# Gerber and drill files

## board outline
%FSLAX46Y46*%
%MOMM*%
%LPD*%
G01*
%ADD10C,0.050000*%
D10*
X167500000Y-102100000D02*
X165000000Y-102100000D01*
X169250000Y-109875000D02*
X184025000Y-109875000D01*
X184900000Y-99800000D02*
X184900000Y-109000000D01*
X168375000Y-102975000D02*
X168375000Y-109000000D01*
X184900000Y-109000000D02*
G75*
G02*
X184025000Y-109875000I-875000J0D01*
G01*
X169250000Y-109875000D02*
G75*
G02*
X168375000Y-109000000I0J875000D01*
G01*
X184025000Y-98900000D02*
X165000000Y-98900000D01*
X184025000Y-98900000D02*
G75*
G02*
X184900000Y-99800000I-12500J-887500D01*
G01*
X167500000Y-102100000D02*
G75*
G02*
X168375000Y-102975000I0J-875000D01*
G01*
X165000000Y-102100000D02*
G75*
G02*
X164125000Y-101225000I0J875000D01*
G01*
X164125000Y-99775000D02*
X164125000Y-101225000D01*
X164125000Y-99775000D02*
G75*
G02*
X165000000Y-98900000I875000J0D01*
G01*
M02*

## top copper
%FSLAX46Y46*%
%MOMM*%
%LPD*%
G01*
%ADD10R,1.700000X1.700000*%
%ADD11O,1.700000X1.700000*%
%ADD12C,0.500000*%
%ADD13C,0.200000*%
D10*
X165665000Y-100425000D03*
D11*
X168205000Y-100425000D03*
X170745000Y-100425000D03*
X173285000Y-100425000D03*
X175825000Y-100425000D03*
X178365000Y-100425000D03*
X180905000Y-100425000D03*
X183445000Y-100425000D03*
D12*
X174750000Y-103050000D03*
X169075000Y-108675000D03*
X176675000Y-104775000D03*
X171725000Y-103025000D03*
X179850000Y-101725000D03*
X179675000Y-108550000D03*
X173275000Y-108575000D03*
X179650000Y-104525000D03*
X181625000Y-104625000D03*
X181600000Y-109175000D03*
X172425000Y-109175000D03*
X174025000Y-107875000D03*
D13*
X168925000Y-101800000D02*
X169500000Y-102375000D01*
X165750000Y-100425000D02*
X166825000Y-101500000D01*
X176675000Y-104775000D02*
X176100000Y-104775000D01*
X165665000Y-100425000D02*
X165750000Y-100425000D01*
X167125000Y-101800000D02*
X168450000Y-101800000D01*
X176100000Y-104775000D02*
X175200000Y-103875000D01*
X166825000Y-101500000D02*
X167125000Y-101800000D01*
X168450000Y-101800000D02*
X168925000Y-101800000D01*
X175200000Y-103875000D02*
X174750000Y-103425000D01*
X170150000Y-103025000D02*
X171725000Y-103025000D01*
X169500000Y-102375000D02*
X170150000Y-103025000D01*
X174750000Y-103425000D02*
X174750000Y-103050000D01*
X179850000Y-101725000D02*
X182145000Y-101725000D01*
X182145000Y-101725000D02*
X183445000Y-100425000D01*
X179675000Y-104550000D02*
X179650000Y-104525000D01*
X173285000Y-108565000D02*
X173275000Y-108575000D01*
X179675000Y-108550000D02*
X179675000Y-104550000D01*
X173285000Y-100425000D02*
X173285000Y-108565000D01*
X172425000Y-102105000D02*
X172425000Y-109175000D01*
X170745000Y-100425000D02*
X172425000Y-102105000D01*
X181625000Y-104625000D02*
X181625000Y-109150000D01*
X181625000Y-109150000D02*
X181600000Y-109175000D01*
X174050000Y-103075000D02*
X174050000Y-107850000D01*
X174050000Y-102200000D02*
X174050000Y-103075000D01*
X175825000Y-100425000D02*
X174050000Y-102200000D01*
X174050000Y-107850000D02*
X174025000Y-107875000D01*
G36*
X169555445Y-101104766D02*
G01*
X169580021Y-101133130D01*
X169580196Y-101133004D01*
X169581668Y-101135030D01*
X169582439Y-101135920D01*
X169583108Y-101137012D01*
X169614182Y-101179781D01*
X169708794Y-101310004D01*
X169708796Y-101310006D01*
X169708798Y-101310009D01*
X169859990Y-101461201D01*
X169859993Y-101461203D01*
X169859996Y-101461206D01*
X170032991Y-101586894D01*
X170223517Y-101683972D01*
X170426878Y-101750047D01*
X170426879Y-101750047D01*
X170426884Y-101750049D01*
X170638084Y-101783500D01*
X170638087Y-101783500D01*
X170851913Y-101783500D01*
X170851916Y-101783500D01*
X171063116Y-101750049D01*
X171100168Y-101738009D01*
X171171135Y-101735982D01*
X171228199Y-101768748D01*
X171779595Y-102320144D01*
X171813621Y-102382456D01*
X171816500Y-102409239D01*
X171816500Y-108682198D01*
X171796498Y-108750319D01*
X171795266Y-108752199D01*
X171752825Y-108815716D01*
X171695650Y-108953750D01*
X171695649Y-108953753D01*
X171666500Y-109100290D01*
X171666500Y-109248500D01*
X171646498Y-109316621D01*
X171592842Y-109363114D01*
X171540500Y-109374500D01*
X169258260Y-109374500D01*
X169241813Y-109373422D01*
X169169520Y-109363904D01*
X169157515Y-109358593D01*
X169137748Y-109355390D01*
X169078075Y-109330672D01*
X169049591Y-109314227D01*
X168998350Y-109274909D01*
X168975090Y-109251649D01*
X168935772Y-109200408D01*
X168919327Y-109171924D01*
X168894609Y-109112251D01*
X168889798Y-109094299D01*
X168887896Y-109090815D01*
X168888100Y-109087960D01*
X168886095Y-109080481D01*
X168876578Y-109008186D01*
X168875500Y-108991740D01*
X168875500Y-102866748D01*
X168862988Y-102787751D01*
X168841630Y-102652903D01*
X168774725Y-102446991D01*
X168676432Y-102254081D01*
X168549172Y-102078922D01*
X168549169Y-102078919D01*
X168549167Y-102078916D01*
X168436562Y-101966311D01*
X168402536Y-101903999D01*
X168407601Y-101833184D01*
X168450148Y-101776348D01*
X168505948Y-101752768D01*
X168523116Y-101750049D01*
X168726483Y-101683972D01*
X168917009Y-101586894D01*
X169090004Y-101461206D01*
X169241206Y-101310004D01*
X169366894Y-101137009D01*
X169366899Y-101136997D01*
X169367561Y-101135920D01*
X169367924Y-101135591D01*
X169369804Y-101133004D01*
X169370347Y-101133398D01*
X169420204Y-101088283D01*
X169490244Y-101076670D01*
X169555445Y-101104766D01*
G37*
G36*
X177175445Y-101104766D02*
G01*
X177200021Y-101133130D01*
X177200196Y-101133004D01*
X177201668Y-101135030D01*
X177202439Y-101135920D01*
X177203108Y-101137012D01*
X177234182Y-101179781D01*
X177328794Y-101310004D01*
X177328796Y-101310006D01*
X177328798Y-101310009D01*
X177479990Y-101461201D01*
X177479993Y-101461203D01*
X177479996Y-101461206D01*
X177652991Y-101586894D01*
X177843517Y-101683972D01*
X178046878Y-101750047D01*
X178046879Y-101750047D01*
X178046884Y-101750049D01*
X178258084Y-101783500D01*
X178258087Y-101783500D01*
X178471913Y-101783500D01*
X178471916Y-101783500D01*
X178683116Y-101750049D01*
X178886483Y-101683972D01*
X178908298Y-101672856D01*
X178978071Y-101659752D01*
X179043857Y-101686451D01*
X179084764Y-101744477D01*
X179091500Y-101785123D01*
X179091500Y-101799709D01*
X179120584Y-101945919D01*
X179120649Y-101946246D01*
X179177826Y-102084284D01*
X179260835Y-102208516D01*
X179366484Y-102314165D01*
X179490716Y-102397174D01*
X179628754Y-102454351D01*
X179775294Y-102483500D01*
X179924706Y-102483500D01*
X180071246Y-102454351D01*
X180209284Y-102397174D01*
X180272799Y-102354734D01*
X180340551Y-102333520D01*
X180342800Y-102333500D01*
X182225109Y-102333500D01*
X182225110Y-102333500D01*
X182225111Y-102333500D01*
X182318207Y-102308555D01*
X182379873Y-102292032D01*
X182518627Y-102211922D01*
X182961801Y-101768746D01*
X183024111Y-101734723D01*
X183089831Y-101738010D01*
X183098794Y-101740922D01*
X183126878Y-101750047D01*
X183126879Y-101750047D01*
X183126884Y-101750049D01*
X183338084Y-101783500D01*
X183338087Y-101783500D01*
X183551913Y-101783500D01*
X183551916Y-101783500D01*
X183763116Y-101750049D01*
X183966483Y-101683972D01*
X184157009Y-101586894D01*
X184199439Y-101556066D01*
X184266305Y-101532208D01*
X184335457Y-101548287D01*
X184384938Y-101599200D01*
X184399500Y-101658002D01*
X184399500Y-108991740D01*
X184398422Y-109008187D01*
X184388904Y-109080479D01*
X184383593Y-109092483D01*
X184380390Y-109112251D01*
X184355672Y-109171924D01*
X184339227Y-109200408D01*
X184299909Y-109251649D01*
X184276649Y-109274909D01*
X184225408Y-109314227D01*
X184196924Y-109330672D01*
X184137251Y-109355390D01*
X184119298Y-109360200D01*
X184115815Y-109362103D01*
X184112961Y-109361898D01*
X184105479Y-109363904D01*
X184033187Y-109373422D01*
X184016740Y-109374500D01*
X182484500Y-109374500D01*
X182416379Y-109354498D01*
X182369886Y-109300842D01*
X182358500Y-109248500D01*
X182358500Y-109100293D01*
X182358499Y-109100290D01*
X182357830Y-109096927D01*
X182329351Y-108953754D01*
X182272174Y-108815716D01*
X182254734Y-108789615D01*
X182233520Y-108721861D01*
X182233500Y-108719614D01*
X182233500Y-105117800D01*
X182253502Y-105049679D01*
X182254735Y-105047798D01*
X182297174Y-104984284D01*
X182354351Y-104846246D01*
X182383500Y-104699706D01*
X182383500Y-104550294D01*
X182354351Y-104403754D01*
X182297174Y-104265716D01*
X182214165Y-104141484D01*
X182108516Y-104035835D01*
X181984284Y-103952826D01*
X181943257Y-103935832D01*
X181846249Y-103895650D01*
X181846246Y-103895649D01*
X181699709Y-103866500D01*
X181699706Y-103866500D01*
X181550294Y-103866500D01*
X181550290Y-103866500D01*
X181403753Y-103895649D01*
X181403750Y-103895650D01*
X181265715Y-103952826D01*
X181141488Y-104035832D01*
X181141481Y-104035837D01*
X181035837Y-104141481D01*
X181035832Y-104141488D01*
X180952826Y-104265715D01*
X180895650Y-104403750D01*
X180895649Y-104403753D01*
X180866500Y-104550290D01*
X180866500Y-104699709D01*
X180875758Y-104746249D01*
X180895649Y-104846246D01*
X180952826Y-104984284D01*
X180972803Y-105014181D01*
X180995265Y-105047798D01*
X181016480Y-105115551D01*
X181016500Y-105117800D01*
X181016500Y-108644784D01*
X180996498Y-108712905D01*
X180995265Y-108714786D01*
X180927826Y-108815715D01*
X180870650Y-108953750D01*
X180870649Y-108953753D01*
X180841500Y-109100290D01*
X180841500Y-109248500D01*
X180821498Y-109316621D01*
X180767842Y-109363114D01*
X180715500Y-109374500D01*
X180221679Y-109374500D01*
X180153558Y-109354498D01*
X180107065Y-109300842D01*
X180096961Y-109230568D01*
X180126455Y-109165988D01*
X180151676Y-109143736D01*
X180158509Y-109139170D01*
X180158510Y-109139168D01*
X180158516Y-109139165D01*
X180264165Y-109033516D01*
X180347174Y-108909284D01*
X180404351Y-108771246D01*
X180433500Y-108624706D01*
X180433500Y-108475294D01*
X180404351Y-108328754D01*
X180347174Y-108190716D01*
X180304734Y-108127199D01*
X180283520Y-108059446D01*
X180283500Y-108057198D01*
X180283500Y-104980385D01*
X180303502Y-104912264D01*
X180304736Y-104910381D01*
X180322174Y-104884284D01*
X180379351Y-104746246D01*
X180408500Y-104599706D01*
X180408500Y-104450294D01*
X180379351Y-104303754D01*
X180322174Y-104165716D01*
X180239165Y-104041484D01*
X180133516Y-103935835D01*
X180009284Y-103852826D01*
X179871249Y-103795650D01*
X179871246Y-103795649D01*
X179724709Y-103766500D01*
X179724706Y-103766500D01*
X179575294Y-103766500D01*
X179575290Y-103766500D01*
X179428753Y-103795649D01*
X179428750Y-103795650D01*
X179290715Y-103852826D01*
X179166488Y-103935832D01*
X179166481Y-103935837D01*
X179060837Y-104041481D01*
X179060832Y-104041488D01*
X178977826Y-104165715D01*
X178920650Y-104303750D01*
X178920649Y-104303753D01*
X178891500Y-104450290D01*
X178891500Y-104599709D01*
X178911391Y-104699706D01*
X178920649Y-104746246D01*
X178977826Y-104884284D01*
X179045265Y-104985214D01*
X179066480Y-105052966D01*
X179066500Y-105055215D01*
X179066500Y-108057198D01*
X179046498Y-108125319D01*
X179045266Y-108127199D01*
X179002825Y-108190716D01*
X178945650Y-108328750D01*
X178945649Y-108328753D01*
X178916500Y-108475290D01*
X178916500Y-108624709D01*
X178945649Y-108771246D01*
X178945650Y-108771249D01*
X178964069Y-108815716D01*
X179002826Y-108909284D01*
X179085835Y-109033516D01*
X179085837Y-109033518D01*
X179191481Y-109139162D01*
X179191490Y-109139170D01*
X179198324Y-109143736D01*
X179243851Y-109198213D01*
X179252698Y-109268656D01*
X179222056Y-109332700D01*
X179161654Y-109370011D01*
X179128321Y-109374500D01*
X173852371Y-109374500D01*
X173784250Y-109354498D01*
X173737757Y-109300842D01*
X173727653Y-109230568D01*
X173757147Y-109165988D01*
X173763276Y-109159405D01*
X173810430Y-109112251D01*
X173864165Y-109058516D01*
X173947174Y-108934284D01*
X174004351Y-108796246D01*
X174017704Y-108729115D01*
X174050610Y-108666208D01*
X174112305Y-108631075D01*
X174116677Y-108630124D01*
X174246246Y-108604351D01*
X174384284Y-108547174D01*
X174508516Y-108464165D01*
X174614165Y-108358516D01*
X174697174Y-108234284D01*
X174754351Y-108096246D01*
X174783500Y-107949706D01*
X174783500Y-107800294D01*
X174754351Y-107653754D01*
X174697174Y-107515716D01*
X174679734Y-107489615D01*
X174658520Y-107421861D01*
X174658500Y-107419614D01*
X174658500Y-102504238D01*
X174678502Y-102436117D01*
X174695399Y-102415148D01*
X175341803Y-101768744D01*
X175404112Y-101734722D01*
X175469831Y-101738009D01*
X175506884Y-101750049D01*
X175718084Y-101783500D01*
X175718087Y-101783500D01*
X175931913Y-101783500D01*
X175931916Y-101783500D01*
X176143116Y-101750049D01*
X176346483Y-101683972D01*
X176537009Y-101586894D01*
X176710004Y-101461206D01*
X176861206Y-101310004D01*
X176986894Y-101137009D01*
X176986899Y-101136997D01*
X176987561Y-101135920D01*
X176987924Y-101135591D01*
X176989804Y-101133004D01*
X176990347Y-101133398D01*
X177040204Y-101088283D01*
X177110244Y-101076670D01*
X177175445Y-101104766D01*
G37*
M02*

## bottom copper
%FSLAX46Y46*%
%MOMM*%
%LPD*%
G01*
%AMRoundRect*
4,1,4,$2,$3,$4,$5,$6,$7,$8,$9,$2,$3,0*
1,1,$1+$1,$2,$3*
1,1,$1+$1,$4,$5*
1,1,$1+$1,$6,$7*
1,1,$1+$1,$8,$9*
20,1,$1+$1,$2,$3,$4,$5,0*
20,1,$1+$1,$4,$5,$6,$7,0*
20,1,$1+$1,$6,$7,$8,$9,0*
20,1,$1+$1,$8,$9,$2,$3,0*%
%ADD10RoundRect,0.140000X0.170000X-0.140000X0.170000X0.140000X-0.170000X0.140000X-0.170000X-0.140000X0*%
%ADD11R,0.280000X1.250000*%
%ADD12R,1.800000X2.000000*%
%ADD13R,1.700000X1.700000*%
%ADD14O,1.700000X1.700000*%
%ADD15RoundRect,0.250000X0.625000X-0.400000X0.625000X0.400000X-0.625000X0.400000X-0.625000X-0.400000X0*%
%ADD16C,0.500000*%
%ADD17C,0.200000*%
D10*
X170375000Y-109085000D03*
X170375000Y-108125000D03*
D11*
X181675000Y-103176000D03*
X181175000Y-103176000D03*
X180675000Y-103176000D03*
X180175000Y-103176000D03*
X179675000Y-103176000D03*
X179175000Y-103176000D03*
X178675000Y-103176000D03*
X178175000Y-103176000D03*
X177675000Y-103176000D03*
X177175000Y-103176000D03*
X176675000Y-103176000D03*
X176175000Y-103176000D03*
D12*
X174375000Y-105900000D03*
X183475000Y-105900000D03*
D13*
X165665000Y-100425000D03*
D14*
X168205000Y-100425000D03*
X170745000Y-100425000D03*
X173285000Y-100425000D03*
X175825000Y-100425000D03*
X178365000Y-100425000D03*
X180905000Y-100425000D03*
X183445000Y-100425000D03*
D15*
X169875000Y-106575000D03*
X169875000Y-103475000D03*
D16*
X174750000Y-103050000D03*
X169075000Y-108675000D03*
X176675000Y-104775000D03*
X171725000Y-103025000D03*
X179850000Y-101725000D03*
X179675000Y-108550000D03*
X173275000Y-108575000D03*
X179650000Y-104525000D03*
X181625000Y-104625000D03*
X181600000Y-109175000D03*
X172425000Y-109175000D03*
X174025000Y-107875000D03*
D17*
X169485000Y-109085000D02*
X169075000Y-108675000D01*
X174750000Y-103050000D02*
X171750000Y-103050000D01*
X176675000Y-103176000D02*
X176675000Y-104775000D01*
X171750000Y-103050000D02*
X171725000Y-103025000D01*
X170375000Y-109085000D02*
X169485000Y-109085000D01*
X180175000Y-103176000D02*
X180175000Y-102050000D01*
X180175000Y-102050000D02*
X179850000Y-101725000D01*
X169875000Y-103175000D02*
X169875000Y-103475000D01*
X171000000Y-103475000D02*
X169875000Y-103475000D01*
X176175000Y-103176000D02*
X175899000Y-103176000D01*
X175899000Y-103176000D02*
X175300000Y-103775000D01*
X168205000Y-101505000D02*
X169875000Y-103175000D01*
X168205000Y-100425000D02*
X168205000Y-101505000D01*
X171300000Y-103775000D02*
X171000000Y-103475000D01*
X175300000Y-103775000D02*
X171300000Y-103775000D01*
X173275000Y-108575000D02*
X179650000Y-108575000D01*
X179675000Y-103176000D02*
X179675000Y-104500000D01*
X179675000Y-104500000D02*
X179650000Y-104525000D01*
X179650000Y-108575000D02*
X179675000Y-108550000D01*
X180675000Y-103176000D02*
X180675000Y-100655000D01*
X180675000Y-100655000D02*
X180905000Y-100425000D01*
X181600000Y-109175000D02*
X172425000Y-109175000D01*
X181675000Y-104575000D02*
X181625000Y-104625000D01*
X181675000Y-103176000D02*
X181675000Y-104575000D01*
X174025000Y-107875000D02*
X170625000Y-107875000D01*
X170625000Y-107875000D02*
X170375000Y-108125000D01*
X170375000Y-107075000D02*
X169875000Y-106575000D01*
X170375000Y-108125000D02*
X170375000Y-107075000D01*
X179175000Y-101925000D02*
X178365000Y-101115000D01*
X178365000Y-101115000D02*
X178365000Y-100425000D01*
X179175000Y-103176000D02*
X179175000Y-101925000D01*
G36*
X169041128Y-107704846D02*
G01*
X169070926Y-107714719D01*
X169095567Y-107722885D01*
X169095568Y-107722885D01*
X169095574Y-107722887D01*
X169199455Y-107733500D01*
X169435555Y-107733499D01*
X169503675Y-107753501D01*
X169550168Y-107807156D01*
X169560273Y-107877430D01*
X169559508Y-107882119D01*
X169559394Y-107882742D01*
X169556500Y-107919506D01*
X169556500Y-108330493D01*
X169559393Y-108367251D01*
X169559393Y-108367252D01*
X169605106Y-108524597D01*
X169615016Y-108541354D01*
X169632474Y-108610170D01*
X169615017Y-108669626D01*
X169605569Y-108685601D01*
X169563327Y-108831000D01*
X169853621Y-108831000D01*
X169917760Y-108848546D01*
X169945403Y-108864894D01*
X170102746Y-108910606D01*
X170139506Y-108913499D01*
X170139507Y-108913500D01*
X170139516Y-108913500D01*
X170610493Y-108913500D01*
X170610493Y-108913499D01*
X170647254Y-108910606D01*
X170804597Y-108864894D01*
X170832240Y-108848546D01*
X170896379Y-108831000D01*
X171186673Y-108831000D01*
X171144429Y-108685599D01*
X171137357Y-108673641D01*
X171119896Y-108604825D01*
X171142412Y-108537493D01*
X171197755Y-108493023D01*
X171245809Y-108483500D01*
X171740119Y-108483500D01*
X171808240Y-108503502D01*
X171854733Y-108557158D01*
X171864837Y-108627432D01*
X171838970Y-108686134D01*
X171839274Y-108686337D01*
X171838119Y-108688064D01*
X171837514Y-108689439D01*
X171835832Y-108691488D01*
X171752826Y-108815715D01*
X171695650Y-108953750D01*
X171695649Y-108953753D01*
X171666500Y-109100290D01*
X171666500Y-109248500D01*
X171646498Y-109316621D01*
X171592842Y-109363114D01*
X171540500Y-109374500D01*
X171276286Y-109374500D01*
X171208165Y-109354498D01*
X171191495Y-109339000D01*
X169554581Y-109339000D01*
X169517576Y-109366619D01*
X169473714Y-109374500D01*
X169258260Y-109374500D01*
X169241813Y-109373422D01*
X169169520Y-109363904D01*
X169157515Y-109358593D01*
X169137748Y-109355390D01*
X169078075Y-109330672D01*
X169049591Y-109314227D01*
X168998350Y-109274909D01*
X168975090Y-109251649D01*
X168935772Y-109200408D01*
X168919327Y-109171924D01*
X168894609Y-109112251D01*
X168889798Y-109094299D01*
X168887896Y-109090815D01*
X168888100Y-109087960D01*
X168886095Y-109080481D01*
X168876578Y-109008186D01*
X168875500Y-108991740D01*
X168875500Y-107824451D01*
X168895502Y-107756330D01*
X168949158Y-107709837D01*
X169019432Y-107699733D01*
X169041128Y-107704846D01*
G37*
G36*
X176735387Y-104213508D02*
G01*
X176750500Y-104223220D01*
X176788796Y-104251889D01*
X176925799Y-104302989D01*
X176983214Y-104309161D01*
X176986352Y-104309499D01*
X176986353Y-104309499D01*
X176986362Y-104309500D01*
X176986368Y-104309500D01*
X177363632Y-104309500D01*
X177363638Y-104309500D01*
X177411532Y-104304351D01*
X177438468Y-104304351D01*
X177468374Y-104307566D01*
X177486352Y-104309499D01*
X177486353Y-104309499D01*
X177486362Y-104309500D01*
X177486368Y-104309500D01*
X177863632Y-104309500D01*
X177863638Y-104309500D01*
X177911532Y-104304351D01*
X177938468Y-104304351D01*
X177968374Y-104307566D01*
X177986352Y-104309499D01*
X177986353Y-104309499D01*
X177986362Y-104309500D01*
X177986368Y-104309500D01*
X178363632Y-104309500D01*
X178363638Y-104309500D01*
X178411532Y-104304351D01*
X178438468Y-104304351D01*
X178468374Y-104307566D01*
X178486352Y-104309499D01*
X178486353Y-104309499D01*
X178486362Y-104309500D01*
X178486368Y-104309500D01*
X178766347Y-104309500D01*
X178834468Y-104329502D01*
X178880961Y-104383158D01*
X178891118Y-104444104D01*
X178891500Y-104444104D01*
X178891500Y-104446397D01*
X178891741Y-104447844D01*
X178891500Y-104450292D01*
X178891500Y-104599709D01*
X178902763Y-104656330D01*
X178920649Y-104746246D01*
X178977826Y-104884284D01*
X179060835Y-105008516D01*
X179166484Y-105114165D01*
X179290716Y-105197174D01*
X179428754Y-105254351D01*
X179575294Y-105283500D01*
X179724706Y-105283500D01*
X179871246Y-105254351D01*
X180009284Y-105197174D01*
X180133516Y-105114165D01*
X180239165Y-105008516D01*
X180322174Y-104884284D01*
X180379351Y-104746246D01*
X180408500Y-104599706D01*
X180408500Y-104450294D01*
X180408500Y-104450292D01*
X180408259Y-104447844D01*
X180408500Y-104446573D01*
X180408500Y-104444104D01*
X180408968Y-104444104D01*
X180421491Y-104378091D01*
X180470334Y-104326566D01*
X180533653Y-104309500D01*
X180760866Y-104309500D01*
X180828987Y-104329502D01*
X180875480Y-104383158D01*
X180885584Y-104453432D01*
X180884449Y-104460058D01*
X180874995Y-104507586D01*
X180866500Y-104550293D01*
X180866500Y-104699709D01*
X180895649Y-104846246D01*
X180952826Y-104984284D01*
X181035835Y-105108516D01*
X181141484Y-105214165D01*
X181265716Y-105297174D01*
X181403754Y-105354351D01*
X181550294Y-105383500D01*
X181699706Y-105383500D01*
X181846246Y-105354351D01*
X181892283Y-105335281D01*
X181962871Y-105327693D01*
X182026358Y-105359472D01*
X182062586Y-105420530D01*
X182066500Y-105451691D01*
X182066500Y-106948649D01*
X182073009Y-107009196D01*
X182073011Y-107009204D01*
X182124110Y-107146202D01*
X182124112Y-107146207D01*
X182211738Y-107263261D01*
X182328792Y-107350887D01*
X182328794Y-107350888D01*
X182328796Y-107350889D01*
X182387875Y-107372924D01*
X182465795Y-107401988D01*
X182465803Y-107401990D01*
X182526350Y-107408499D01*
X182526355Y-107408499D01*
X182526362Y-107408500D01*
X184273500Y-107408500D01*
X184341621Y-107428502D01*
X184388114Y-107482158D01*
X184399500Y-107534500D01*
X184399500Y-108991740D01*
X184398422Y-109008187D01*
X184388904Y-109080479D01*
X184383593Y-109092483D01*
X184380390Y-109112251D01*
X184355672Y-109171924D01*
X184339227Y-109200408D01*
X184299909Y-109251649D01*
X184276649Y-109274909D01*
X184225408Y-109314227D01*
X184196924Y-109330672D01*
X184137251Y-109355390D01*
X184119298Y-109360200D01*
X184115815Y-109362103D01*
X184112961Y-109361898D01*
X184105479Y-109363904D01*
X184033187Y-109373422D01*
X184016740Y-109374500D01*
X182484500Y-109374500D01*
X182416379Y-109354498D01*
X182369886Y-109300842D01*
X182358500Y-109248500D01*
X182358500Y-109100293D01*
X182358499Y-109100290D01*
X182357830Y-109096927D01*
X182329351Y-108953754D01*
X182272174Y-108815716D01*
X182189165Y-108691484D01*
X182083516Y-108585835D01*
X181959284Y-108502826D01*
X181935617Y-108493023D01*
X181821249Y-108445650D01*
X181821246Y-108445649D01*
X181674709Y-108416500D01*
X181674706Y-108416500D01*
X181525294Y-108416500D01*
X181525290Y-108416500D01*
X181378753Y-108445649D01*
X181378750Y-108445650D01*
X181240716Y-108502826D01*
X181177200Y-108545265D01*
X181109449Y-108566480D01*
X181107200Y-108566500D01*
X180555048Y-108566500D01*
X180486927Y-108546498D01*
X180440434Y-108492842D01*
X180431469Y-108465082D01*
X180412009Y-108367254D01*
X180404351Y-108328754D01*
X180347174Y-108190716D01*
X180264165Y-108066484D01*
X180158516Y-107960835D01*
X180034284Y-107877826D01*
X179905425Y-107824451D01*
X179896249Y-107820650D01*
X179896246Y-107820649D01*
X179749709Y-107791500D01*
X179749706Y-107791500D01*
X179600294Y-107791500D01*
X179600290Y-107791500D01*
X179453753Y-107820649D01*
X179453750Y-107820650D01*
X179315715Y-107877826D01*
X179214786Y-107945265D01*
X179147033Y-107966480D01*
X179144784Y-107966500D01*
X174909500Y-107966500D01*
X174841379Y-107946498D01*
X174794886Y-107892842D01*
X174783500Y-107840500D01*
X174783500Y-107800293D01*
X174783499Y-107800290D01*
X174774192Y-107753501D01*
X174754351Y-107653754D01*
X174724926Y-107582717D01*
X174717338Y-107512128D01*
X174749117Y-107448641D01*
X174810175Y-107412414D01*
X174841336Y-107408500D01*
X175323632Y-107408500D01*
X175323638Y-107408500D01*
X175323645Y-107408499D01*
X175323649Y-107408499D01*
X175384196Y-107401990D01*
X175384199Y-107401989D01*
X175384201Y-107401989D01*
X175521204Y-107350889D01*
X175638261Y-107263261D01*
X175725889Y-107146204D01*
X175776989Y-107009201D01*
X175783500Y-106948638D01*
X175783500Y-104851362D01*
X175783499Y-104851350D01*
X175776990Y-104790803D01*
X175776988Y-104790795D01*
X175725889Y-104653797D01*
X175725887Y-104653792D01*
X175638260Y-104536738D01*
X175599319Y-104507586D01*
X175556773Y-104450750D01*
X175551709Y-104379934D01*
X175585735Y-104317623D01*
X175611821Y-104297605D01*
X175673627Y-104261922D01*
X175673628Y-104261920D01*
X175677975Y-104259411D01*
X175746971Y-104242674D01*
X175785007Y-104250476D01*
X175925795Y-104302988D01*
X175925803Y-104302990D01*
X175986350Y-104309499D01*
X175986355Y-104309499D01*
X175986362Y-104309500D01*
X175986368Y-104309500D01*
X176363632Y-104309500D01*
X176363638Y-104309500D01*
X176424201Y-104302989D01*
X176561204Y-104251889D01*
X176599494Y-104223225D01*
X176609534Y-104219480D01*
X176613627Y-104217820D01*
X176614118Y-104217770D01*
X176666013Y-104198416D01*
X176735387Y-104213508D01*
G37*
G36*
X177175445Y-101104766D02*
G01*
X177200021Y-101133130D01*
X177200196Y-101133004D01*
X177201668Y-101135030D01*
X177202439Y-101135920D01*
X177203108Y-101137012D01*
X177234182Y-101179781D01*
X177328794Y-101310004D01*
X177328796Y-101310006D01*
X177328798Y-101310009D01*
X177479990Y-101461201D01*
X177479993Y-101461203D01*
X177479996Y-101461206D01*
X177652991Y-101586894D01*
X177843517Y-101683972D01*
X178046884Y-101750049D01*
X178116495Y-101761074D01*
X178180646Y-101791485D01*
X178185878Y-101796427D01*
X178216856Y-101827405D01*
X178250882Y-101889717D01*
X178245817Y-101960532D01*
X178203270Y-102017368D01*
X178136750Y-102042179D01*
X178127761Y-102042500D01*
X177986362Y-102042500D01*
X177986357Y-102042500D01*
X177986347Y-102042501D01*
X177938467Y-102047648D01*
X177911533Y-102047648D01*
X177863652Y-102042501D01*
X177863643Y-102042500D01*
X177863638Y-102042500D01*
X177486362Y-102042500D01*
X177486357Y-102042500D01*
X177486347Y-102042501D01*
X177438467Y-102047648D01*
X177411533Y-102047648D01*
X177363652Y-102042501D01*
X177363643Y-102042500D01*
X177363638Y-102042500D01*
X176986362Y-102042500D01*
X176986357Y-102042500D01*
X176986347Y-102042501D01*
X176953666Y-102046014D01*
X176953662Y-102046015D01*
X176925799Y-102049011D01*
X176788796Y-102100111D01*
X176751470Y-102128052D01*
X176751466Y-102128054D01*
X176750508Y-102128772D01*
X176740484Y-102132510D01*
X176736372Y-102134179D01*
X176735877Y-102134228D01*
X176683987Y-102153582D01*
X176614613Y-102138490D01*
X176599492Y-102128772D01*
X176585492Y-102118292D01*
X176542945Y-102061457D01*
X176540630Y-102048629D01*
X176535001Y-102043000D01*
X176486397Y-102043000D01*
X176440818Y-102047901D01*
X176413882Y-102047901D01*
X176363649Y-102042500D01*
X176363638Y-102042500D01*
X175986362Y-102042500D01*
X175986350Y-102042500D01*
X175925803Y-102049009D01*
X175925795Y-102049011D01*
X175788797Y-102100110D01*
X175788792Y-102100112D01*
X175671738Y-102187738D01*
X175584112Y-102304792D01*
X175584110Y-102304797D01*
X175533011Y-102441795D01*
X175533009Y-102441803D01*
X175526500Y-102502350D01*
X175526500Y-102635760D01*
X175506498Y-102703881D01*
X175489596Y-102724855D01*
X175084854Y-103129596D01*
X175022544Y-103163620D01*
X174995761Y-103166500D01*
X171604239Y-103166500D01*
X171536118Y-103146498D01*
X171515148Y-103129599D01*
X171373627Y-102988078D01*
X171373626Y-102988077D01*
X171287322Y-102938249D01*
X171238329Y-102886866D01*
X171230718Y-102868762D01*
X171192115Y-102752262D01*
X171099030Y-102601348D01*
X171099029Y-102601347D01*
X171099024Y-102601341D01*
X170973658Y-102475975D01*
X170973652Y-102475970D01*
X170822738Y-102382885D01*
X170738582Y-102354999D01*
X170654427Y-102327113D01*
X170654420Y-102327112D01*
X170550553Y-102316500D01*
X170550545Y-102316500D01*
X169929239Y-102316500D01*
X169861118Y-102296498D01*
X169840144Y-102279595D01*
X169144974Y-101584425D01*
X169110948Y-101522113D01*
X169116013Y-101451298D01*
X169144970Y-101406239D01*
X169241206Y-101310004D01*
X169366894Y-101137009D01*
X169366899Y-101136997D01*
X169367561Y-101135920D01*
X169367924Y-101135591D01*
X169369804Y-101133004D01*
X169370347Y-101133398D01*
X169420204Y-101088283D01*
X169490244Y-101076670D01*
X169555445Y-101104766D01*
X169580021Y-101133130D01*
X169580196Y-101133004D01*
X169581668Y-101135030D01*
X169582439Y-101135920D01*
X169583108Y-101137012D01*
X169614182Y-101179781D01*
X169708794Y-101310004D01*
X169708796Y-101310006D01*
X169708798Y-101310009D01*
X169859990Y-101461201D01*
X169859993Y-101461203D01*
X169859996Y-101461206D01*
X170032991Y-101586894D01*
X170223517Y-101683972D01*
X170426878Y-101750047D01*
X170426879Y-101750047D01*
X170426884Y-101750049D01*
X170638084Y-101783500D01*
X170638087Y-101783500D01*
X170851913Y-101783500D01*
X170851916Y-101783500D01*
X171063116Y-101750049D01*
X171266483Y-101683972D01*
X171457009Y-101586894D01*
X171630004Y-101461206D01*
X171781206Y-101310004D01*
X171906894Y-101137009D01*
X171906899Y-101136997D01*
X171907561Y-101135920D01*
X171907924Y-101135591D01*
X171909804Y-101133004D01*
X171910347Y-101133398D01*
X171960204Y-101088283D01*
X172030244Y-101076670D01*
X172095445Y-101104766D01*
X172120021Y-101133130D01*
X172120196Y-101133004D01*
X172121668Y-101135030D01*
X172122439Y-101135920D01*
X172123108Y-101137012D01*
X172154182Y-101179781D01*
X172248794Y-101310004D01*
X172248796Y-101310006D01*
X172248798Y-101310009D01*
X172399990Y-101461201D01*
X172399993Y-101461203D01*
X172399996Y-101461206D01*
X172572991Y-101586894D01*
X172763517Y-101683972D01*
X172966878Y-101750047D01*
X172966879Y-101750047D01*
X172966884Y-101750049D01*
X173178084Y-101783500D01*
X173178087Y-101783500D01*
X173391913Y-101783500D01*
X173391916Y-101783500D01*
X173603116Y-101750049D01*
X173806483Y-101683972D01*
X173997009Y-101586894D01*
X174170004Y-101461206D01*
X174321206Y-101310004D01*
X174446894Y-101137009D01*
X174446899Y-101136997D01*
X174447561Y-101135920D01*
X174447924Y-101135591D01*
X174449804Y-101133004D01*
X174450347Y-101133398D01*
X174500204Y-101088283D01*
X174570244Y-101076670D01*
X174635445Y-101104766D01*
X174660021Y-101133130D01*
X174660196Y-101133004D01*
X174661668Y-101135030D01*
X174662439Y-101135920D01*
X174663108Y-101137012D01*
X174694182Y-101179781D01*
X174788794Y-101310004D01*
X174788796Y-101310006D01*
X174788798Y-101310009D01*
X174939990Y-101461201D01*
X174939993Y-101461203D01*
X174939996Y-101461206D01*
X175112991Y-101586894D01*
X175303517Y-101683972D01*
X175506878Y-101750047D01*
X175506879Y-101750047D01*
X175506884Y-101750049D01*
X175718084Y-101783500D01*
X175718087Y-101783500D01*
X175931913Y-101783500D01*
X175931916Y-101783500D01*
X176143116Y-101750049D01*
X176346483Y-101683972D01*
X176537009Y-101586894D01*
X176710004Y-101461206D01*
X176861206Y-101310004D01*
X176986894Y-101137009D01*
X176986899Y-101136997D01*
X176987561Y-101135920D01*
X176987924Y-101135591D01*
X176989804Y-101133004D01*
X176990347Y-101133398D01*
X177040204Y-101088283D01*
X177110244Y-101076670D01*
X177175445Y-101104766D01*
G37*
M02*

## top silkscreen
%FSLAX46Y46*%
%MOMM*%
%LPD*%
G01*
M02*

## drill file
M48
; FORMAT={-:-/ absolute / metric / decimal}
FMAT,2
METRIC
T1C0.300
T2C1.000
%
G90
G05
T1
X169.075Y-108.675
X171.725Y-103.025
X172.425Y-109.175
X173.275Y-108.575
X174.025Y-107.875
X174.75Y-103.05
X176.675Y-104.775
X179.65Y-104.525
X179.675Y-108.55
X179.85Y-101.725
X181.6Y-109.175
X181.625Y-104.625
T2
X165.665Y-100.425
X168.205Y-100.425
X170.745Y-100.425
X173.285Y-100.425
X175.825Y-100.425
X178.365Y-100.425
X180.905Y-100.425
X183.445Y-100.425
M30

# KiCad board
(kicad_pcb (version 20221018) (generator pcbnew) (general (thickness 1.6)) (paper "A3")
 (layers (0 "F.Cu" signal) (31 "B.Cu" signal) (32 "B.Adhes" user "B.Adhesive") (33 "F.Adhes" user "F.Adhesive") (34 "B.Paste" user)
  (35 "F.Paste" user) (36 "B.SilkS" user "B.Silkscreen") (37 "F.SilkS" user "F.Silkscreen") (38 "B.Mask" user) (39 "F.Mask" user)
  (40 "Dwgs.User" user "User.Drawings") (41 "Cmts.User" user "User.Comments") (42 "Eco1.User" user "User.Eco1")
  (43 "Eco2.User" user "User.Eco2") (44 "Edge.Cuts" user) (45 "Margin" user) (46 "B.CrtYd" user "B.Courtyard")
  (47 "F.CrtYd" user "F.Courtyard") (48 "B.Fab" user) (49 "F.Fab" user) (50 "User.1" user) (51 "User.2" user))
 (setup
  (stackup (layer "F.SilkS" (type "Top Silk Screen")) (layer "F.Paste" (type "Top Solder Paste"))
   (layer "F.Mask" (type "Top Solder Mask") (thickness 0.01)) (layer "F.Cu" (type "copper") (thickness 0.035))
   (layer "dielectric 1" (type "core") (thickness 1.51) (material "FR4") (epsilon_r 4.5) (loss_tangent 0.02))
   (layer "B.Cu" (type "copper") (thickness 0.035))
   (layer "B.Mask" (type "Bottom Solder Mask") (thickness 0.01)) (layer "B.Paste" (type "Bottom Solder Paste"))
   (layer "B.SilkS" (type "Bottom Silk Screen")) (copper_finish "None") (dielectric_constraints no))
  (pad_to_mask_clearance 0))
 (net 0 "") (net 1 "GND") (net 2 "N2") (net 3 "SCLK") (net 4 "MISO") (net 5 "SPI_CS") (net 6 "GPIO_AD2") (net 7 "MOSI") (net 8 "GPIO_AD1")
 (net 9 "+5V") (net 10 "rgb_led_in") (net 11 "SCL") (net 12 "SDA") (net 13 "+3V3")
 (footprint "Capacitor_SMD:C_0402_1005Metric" (layer "B.Cu") (at 170.375 108.605 90)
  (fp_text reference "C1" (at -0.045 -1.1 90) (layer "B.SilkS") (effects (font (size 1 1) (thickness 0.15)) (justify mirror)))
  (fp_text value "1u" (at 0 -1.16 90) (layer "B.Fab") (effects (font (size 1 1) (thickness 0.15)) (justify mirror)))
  (pad "1" smd roundrect (at -0.48 0 90) (size 0.56 0.62) (layers "B.Cu" "B.Paste" "B.Mask") (roundrect_rratio 0.25) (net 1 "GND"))
  (pad "2" smd roundrect (at 0.48 0 90) (size 0.56 0.62) (layers "B.Cu" "B.Paste" "B.Mask") (roundrect_rratio 0.25) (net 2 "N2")))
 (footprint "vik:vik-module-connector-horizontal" (layer "B.Cu") (at 178.925 105.214 180)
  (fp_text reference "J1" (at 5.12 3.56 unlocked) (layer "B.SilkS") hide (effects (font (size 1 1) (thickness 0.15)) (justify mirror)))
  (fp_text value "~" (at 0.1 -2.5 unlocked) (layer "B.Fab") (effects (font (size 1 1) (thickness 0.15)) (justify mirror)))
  (pad "1" smd rect (at -2.75 2.038 180) (size 0.28 1.25) (layers "B.Cu" "B.Paste" "B.Mask") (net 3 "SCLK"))
  (pad "2" smd rect (at -2.25 2.038 180) (size 0.28 1.25) (layers "B.Cu" "B.Paste" "B.Mask") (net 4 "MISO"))
  (pad "3" smd rect (at -1.75 2.038 180) (size 0.28 1.25) (layers "B.Cu" "B.Paste" "B.Mask") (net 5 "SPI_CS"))
  (pad "4" smd rect (at -1.25 2.038 180) (size 0.28 1.25) (layers "B.Cu" "B.Paste" "B.Mask") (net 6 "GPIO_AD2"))
  (pad "5" smd rect (at -0.75 2.038 180) (size 0.28 1.25) (layers "B.Cu" "B.Paste" "B.Mask") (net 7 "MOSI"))
  (pad "6" smd rect (at -0.25 2.038 180) (size 0.28 1.25) (layers "B.Cu" "B.Paste" "B.Mask") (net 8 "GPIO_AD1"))
  (pad "7" smd rect (at 0.25 2.038 180) (size 0.28 1.25) (layers "B.Cu" "B.Paste" "B.Mask") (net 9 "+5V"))
  (pad "8" smd rect (at 0.75 2.038 180) (size 0.28 1.25) (layers "B.Cu" "B.Paste" "B.Mask") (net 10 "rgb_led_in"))
  (pad "9" smd rect (at 1.25 2.038 180) (size 0.28 1.25) (layers "B.Cu" "B.Paste" "B.Mask") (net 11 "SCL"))
  (pad "10" smd rect (at 1.75 2.038 180) (size 0.28 1.25) (layers "B.Cu" "B.Paste" "B.Mask") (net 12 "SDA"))
  (pad "11" smd rect (at 2.25 2.038 180) (size 0.28 1.25) (layers "B.Cu" "B.Paste" "B.Mask") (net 1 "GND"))
  (pad "12" smd rect (at 2.75 2.038 180) (size 0.28 1.25) (layers "B.Cu" "B.Paste" "B.Mask") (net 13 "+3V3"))
  (pad "13" smd rect (at 4.55 -0.686 180) (size 1.8 2) (layers "B.Cu" "B.Paste" "B.Mask"))
  (pad "14" smd rect (at -4.55 -0.686 180) (size 1.8 2) (layers "B.Cu" "B.Paste" "B.Mask")))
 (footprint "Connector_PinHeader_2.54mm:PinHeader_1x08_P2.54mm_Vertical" (layer "B.Cu") (at 165.665 100.425 -90)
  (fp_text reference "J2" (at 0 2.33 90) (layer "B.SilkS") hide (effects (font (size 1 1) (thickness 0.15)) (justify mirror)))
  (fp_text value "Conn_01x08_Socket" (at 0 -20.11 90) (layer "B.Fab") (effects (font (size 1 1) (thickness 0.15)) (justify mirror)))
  (pad "1" thru_hole rect (at 0 0 270) (size 1.7 1.7) (drill 1) (layers "*.Cu" "*.Mask") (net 1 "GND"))
  (pad "2" thru_hole oval (at 0 -2.54 270) (size 1.7 1.7) (drill 1) (layers "*.Cu" "*.Mask") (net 13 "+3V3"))
  (pad "3" thru_hole oval (at 0 -5.08 270) (size 1.7 1.7) (drill 1) (layers "*.Cu" "*.Mask") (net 3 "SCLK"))
  (pad "4" thru_hole oval (at 0 -7.62 270) (size 1.7 1.7) (drill 1) (layers "*.Cu" "*.Mask") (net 7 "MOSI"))
  (pad "5" thru_hole oval (at 0 -10.16 270) (size 1.7 1.7) (drill 1) (layers "*.Cu" "*.Mask") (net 2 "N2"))
  (pad "6" thru_hole oval (at 0 -12.7 270) (size 1.7 1.7) (drill 1) (layers "*.Cu" "*.Mask") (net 8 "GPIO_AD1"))
  (pad "7" thru_hole oval (at 0 -15.24 270) (size 1.7 1.7) (drill 1) (layers "*.Cu" "*.Mask") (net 5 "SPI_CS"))
  (pad "8" thru_hole oval (at 0 -17.78 270) (size 1.7 1.7) (drill 1) (layers "*.Cu" "*.Mask") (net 6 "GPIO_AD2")))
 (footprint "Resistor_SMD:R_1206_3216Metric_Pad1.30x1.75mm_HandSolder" (layer "B.Cu") (at 169.875 105.025 90)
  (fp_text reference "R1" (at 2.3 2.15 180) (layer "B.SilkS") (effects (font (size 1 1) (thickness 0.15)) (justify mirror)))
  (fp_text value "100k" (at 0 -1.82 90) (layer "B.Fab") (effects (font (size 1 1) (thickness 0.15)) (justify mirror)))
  (pad "1" smd roundrect (at -1.55 0 90) (size 1.3 1.75) (layers "B.Cu" "B.Paste" "B.Mask") (roundrect_rratio 0.1923076923) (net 2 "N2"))
  (pad "2" smd roundrect (at 1.55 0 90) (size 1.3 1.75) (layers "B.Cu" "B.Paste" "B.Mask") (roundrect_rratio 0.1923076923) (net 13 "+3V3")))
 (gr_line (start 167.5 102.1) (end 165 102.1) (stroke (width 0.05) (type solid)) (layer "Edge.Cuts"))
 (gr_line (start 169.25 109.875) (end 184.025 109.875) (stroke (width 0.05) (type solid)) (layer "Edge.Cuts"))
 (gr_line (start 184.9 99.8) (end 184.9 109) (stroke (width 0.05) (type solid)) (layer "Edge.Cuts"))
 (gr_line (start 168.375 102.975) (end 168.375 109) (stroke (width 0.05) (type solid)) (layer "Edge.Cuts"))
 (gr_arc (start 184.9 109) (mid 184.643718 109.618718) (end 184.025 109.875) (stroke (width 0.05) (type solid)) (layer "Edge.Cuts"))
 (gr_arc (start 169.25 109.875) (mid 168.631282 109.618718) (end 168.375 109) (stroke (width 0.05) (type solid)) (layer "Edge.Cuts"))
 (gr_line (start 184.025 98.9) (end 165 98.9) (stroke (width 0.05) (type solid)) (layer "Edge.Cuts"))
 (gr_arc (start 184.025 98.9) (mid 184.648896 99.168782) (end 184.9 99.8) (stroke (width 0.05) (type solid)) (layer "Edge.Cuts"))
 (gr_arc (start 167.5 102.1) (mid 168.118718 102.356282) (end 168.375 102.975) (stroke (width 0.05) (type solid)) (layer "Edge.Cuts"))
 (gr_arc (start 165 102.1) (mid 164.381282 101.843718) (end 164.125 101.225) (stroke (width 0.05) (type solid)) (layer "Edge.Cuts"))
 (gr_line (start 164.125 99.775) (end 164.125 101.225) (stroke (width 0.05) (type solid)) (layer "Edge.Cuts"))
 (gr_arc (start 164.125 99.775) (mid 164.381282 99.156282) (end 165 98.9) (stroke (width 0.05) (type solid)) (layer "Edge.Cuts"))
 (segment (start 168.925 101.8) (end 169.5 102.375) (width 0.2) (layer "F.Cu") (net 1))
 (segment (start 165.75 100.425) (end 166.825 101.5) (width 0.2) (layer "F.Cu") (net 1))
 (segment (start 176.675 104.775) (end 176.1 104.775) (width 0.2) (layer "F.Cu") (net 1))
 (segment (start 165.665 100.425) (end 165.75 100.425) (width 0.2) (layer "F.Cu") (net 1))
 (segment (start 167.125 101.8) (end 168.45 101.8) (width 0.2) (layer "F.Cu") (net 1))
 (segment (start 176.1 104.775) (end 175.2 103.875) (width 0.2) (layer "F.Cu") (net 1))
 (segment (start 166.825 101.5) (end 167.125 101.8) (width 0.2) (layer "F.Cu") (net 1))
 (segment (start 168.45 101.8) (end 168.925 101.8) (width 0.2) (layer "F.Cu") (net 1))
 (segment (start 175.2 103.875) (end 174.75 103.425) (width 0.2) (layer "F.Cu") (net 1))
 (segment (start 170.15 103.025) (end 171.725 103.025) (width 0.2) (layer "F.Cu") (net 1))
 (segment (start 169.5 102.375) (end 170.15 103.025) (width 0.2) (layer "F.Cu") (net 1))
 (segment (start 174.75 103.425) (end 174.75 103.05) (width 0.2) (layer "F.Cu") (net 1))
 (via (at 174.75 103.05) (size 0.5) (drill 0.3) (layers "F.Cu" "B.Cu") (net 1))
 (via (at 169.075 108.675) (size 0.5) (drill 0.3) (layers "F.Cu" "B.Cu") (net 1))
 (via (at 176.675 104.775) (size 0.5) (drill 0.3) (layers "F.Cu" "B.Cu") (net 1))
 (via (at 171.725 103.025) (size 0.5) (drill 0.3) (layers "F.Cu" "B.Cu") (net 1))
 (segment (start 169.485 109.085) (end 169.075 108.675) (width 0.2) (layer "B.Cu") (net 1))
 (segment (start 174.75 103.05) (end 171.75 103.05) (width 0.2) (layer "B.Cu") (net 1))
 (segment (start 176.675 103.176) (end 176.675 104.775) (width 0.2) (layer "B.Cu") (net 1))
 (segment (start 171.75 103.05) (end 171.725 103.025) (width 0.2) (layer "B.Cu") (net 1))
 (segment (start 170.375 109.085) (end 169.485 109.085) (width 0.2) (layer "B.Cu") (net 1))
 (segment (start 179.85 101.725) (end 182.145 101.725) (width 0.2) (layer "F.Cu") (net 6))
 (segment (start 182.145 101.725) (end 183.445 100.425) (width 0.2) (layer "F.Cu") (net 6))
 (via (at 179.85 101.725) (size 0.5) (drill 0.3) (layers "F.Cu" "B.Cu") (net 6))
 (segment (start 180.175 103.176) (end 180.175 102.05) (width 0.2) (layer "B.Cu") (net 6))
 (segment (start 180.175 102.05) (end 179.85 101.725) (width 0.2) (layer "B.Cu") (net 6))
 (segment (start 169.875 103.175) (end 169.875 103.475) (width 0.2) (layer "B.Cu") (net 13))
 (segment (start 171 103.475) (end 169.875 103.475) (width 0.2) (layer "B.Cu") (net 13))
 (segment (start 176.175 103.176) (end 175.899 103.176) (width 0.2) (layer "B.Cu") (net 13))
 (segment (start 175.899 103.176) (end 175.3 103.775) (width 0.2) (layer "B.Cu") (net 13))
 (segment (start 168.205 101.505) (end 169.875 103.175) (width 0.2) (layer "B.Cu") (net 13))
 (segment (start 168.205 100.425) (end 168.205 101.505) (width 0.2) (layer "B.Cu") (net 13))
 (segment (start 171.3 103.775) (end 171 103.475) (width 0.2) (layer "B.Cu") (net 13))
 (segment (start 175.3 103.775) (end 171.3 103.775) (width 0.2) (layer "B.Cu") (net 13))
 (segment (start 179.675 104.55) (end 179.65 104.525) (width 0.2) (layer "F.Cu") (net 7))
 (segment (start 173.285 108.565) (end 173.275 108.575) (width 0.2) (layer "F.Cu") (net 7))
 (segment (start 179.675 108.55) (end 179.675 104.55) (width 0.2) (layer "F.Cu") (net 7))
 (segment (start 173.285 100.425) (end 173.285 108.565) (width 0.2) (layer "F.Cu") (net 7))
 (via (at 179.675 108.55) (size 0.5) (drill 0.3) (layers "F.Cu" "B.Cu") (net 7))
 (via (at 173.275 108.575) (size 0.5) (drill 0.3) (layers "F.Cu" "B.Cu") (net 7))
 (via (at 179.65 104.525) (size 0.5) (drill 0.3) (layers "F.Cu" "B.Cu") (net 7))
 (segment (start 173.275 108.575) (end 179.65 108.575) (width 0.2) (layer "B.Cu") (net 7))
 (segment (start 179.675 103.176) (end 179.675 104.5) (width 0.2) (layer "B.Cu") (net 7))
 (segment (start 179.675 104.5) (end 179.65 104.525) (width 0.2) (layer "B.Cu") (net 7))
 (segment (start 179.65 108.575) (end 179.675 108.55) (width 0.2) (layer "B.Cu") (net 7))
 (segment (start 180.675 103.176) (end 180.675 100.655) (width 0.2) (layer "B.Cu") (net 5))
 (segment (start 180.675 100.655) (end 180.905 100.425) (width 0.2) (layer "B.Cu") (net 5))
 (segment (start 172.425 102.105) (end 172.425 109.175) (width 0.2) (layer "F.Cu") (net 3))
 (segment (start 170.745 100.425) (end 172.425 102.105) (width 0.2) (layer "F.Cu") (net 3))
 (segment (start 181.625 104.625) (end 181.625 109.15) (width 0.2) (layer "F.Cu") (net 3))
 (segment (start 181.625 109.15) (end 181.6 109.175) (width 0.2) (layer "F.Cu") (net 3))
 (via (at 181.625 104.625) (size 0.5) (drill 0.3) (layers "F.Cu" "B.Cu") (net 3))
 (via (at 181.6 109.175) (size 0.5) (drill 0.3) (layers "F.Cu" "B.Cu") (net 3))
 (via (at 172.425 109.175) (size 0.5) (drill 0.3) (layers "F.Cu" "B.Cu") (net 3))
 (segment (start 181.6 109.175) (end 172.425 109.175) (width 0.2) (layer "B.Cu") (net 3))
 (segment (start 181.675 104.575) (end 181.625 104.625) (width 0.2) (layer "B.Cu") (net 3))
 (segment (start 181.675 103.176) (end 181.675 104.575) (width 0.2) (layer "B.Cu") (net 3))
 (segment (start 174.05 103.075) (end 174.05 107.85) (width 0.2) (layer "F.Cu") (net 2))
 (segment (start 174.05 102.2) (end 174.05 103.075) (width 0.2) (layer "F.Cu") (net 2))
 (segment (start 175.825 100.425) (end 174.05 102.2) (width 0.2) (layer "F.Cu") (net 2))
 (segment (start 174.05 107.85) (end 174.025 107.875) (width 0.2) (layer "F.Cu") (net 2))
 (via (at 174.025 107.875) (size 0.5) (drill 0.3) (layers "F.Cu" "B.Cu") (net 2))
 (segment (start 174.025 107.875) (end 170.625 107.875) (width 0.2) (layer "B.Cu") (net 2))
 (segment (start 170.625 107.875) (end 170.375 108.125) (width 0.2) (layer "B.Cu") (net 2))
 (segment (start 170.375 107.075) (end 169.875 106.575) (width 0.2) (layer "B.Cu") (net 2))
 (segment (start 170.375 108.125) (end 170.375 107.075) (width 0.2) (layer "B.Cu") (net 2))
 (segment (start 179.175 101.925) (end 178.365 101.115) (width 0.2) (layer "B.Cu") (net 8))
 (segment (start 178.365 101.115) (end 178.365 100.425) (width 0.2) (layer "B.Cu") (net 8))
 (segment (start 179.175 103.176) (end 179.175 101.925) (width 0.2) (layer "B.Cu") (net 8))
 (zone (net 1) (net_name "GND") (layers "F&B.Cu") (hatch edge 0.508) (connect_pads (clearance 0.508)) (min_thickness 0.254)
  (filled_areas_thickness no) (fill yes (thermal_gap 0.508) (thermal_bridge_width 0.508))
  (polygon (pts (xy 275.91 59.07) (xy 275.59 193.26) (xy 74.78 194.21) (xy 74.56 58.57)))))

